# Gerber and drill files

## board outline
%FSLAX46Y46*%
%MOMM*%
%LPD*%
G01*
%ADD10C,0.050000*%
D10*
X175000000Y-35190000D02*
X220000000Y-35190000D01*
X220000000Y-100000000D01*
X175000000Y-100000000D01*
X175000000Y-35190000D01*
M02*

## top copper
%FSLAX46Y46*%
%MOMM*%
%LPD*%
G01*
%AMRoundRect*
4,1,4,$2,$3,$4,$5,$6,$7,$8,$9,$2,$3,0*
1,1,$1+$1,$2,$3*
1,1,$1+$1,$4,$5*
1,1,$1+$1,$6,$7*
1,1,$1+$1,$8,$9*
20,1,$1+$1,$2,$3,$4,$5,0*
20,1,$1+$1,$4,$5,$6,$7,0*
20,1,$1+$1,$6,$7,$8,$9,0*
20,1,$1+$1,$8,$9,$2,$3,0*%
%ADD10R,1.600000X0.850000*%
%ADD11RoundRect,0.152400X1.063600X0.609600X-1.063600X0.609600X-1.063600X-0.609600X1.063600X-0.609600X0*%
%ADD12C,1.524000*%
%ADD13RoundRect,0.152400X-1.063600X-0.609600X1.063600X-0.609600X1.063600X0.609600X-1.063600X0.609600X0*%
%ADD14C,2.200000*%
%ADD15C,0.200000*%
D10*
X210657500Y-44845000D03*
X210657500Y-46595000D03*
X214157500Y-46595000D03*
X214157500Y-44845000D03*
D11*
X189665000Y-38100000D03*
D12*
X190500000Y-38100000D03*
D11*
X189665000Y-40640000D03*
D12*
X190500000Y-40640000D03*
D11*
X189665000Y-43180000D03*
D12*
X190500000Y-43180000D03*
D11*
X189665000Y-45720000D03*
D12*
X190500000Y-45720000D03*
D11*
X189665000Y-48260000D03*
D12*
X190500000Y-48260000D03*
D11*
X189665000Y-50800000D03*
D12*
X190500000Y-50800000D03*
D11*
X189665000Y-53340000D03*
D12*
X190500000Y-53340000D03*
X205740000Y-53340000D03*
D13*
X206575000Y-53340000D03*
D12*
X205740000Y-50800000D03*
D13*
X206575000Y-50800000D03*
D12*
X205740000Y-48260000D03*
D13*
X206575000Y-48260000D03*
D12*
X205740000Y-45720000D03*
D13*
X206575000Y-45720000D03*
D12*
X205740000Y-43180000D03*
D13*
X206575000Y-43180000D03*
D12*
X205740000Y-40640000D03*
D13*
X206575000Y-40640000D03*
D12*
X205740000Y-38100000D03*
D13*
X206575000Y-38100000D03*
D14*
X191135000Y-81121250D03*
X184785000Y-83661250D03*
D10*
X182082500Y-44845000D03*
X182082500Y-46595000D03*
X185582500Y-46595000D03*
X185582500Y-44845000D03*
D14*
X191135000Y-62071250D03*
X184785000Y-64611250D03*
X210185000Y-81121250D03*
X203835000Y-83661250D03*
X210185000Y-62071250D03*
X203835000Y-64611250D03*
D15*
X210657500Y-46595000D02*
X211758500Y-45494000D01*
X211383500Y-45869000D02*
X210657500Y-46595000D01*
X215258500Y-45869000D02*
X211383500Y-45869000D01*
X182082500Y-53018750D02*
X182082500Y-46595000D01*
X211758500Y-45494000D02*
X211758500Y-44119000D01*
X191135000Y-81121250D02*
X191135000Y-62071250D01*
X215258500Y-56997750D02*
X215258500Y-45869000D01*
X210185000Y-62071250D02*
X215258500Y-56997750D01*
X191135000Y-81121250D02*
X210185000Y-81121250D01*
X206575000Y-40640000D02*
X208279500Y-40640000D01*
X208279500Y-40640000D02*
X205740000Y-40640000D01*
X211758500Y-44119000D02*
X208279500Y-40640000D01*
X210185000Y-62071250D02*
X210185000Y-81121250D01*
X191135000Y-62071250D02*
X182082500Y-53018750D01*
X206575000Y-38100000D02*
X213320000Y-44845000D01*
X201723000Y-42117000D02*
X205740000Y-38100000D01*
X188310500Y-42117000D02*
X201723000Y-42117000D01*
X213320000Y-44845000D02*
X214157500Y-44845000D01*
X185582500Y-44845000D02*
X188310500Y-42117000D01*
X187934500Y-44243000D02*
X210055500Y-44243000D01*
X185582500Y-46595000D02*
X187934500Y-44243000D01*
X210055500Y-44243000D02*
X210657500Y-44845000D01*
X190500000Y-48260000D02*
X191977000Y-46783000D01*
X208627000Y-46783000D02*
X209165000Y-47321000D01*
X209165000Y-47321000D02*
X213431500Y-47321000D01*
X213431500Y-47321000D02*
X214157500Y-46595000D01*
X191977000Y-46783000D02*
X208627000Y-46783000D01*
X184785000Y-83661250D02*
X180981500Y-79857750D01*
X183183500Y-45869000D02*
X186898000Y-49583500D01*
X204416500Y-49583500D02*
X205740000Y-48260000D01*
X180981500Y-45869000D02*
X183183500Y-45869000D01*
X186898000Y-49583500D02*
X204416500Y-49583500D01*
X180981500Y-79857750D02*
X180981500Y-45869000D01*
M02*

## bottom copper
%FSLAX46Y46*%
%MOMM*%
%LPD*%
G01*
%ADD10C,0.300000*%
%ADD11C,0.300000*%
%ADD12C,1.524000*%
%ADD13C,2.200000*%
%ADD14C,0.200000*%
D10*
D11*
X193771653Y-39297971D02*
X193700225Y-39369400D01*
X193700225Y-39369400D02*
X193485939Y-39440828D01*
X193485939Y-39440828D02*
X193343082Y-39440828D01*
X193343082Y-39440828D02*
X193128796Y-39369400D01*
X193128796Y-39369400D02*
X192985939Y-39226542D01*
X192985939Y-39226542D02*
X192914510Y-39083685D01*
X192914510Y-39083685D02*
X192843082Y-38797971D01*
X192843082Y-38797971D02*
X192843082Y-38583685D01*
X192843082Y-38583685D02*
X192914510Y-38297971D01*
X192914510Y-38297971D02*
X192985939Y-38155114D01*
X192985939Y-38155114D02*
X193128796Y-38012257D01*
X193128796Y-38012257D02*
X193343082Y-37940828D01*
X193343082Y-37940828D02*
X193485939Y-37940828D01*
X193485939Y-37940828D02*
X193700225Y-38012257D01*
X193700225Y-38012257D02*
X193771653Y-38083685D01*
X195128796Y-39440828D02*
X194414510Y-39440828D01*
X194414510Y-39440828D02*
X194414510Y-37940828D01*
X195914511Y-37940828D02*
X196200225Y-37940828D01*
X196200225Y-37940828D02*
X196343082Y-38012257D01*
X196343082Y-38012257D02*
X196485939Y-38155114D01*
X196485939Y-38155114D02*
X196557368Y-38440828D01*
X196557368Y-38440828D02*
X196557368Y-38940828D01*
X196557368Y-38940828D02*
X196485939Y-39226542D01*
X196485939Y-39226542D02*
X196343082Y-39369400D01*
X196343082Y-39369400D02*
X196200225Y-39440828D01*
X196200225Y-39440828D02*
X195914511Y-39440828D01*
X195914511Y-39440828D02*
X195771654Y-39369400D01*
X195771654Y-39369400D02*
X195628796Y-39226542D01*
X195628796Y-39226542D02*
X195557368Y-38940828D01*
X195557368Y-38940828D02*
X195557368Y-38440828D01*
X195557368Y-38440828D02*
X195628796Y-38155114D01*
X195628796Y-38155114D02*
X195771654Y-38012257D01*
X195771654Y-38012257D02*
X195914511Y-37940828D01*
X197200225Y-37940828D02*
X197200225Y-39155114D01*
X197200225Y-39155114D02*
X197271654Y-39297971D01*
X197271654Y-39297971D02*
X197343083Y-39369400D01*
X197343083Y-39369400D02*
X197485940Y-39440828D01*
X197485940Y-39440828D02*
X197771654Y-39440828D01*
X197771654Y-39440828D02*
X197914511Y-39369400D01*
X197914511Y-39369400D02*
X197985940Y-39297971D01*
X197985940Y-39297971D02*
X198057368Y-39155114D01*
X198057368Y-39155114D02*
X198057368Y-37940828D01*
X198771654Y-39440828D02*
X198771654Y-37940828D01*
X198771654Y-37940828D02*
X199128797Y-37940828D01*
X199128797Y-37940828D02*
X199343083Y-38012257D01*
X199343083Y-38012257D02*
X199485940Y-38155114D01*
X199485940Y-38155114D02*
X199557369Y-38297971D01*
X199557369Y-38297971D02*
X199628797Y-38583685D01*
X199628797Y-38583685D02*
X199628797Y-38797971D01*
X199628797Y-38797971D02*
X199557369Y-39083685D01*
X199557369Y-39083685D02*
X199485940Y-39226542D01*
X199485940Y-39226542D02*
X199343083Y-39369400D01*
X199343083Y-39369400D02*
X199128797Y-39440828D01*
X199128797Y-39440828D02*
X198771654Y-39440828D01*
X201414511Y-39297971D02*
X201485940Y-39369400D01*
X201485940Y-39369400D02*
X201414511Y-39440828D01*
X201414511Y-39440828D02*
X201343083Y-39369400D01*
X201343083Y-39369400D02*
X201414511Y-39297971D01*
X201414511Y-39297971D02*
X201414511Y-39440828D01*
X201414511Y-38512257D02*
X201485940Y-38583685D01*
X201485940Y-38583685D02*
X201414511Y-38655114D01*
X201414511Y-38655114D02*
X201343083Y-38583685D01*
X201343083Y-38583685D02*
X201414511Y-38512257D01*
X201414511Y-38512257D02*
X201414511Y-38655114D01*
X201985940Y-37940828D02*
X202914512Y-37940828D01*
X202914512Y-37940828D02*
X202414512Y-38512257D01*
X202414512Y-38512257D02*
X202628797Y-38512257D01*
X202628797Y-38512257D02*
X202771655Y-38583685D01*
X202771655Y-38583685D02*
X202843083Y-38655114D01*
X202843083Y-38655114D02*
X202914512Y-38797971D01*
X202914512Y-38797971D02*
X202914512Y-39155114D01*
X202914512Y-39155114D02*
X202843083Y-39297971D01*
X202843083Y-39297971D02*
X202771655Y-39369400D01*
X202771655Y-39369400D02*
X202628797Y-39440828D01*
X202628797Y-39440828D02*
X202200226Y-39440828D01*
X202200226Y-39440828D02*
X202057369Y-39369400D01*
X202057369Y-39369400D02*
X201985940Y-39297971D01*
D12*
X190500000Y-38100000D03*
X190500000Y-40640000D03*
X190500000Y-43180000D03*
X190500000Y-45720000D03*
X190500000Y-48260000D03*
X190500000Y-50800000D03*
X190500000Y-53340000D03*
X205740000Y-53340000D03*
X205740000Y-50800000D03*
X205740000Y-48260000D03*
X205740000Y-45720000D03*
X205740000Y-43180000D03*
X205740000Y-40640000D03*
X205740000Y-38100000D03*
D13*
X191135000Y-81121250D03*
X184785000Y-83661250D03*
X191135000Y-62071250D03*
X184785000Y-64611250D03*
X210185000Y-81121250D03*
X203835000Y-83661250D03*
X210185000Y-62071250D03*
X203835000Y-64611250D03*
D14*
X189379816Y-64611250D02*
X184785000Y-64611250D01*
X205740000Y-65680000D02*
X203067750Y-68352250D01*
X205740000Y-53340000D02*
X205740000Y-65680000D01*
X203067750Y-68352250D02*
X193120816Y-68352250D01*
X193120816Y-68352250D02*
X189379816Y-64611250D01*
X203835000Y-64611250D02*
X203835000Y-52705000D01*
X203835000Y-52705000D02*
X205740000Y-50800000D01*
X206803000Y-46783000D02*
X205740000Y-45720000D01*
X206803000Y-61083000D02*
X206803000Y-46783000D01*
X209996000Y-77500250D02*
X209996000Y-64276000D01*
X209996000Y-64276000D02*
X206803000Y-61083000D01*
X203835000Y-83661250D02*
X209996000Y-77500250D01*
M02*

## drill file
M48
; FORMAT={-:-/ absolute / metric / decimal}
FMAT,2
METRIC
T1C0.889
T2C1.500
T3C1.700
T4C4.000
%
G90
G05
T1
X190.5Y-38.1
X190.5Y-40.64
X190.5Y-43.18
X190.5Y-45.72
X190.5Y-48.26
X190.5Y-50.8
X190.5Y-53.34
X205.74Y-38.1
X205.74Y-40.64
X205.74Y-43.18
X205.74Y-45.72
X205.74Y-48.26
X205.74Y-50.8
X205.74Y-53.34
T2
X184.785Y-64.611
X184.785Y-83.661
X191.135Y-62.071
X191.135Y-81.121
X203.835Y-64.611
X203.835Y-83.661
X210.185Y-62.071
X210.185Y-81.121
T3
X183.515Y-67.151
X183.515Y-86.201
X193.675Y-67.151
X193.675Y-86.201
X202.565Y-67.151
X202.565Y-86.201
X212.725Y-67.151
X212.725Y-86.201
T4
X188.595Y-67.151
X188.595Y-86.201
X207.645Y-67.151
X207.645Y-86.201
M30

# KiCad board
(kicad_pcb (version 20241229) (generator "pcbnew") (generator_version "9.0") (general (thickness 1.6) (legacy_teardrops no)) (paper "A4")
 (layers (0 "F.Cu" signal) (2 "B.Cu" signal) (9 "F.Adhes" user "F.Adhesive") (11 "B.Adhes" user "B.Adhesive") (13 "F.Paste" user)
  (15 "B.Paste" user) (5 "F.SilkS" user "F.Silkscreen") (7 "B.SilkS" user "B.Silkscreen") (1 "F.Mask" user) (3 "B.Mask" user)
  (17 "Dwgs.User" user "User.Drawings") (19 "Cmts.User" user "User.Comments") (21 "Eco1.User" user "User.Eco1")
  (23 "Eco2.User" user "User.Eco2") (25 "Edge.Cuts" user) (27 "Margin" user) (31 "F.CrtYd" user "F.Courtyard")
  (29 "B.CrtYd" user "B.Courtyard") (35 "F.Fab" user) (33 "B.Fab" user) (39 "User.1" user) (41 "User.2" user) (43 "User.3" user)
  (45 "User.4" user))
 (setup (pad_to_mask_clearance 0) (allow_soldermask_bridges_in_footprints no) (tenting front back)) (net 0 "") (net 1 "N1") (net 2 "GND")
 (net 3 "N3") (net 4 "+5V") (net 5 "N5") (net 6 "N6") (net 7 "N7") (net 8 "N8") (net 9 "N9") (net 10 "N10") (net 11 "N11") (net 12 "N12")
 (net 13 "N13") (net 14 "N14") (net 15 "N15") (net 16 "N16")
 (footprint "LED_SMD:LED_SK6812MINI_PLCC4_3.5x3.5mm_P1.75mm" (layer "F.Cu") (at 212.4075 45.72)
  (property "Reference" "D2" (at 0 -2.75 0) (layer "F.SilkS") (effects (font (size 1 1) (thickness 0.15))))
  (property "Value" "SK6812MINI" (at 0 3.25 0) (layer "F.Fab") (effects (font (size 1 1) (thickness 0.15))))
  (pad "1" smd rect (at -1.75 -0.875) (size 1.6 0.85) (layers "F.Cu" "F.Mask" "F.Paste") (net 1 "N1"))
  (pad "2" smd rect (at -1.75 0.875) (size 1.6 0.85) (layers "F.Cu" "F.Mask" "F.Paste") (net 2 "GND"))
  (pad "3" smd rect (at 1.75 0.875) (size 1.6 0.85) (layers "F.Cu" "F.Mask" "F.Paste") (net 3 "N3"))
  (pad "4" smd rect (at 1.75 -0.875) (size 1.6 0.85) (layers "F.Cu" "F.Mask" "F.Paste") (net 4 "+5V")))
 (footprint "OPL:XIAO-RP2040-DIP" (layer "F.Cu") (at 198.12 45.72)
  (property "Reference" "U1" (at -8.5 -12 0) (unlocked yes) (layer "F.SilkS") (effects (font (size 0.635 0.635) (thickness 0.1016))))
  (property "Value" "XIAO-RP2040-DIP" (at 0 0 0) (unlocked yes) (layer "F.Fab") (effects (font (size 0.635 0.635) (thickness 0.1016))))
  (pad "1" smd roundrect (at -8.455 -7.62 180) (size 2.432 1.524) (layers "F.Cu" "F.Mask") (roundrect_rratio 0.1) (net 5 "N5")
   (thermal_bridge_angle 45))
  (pad "1" thru_hole circle (at -7.62 -7.62 180) (size 1.524 1.524) (drill 0.889) (layers "*.Cu" "*.Mask") (remove_unused_layers no)
   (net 5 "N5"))
  (pad "2" smd roundrect (at -8.455 -5.08 180) (size 2.432 1.524) (layers "F.Cu" "F.Mask") (roundrect_rratio 0.1) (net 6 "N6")
   (thermal_bridge_angle 45))
  (pad "2" thru_hole circle (at -7.62 -5.08 180) (size 1.524 1.524) (drill 0.889) (layers "*.Cu" "*.Mask") (remove_unused_layers no)
   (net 6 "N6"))
  (pad "3" smd roundrect (at -8.455 -2.54 180) (size 2.432 1.524) (layers "F.Cu" "F.Mask") (roundrect_rratio 0.1) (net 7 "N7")
   (thermal_bridge_angle 45))
  (pad "3" thru_hole circle (at -7.62 -2.54 180) (size 1.524 1.524) (drill 0.889) (layers "*.Cu" "*.Mask") (remove_unused_layers no)
   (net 7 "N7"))
  (pad "4" smd roundrect (at -8.455 0 180) (size 2.432 1.524) (layers "F.Cu" "F.Mask") (roundrect_rratio 0.1) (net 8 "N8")
   (thermal_bridge_angle 45))
  (pad "4" thru_hole circle (at -7.62 0 180) (size 1.524 1.524) (drill 0.889) (layers "*.Cu" "*.Mask") (remove_unused_layers no)
   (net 8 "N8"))
  (pad "5" smd roundrect (at -8.455 2.54 180) (size 2.432 1.524) (layers "F.Cu" "F.Mask") (roundrect_rratio 0.1) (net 3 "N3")
   (thermal_bridge_angle 45))
  (pad "5" thru_hole circle (at -7.62 2.54 180) (size 1.524 1.524) (drill 0.889) (layers "*.Cu" "*.Mask") (remove_unused_layers no)
   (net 3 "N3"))
  (pad "6" smd roundrect (at -8.455 5.08 180) (size 2.432 1.524) (layers "F.Cu" "F.Mask") (roundrect_rratio 0.1) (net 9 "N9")
   (thermal_bridge_angle 45))
  (pad "6" thru_hole circle (at -7.62 5.08 180) (size 1.524 1.524) (drill 0.889) (layers "*.Cu" "*.Mask") (remove_unused_layers no)
   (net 9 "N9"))
  (pad "7" smd roundrect (at -8.455 7.62 180) (size 2.432 1.524) (layers "F.Cu" "F.Mask") (roundrect_rratio 0.1) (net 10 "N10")
   (thermal_bridge_angle 45))
  (pad "7" thru_hole circle (at -7.62 7.62 180) (size 1.524 1.524) (drill 0.889) (layers "*.Cu" "*.Mask") (remove_unused_layers no)
   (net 10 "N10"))
  (pad "8" thru_hole circle (at 7.62 7.62) (size 1.524 1.524) (drill 0.889) (layers "*.Cu" "*.Mask") (remove_unused_layers no)
   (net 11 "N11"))
  (pad "8" smd roundrect (at 8.455 7.62) (size 2.432 1.524) (layers "F.Cu" "F.Mask") (roundrect_rratio 0.1) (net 11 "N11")
   (thermal_bridge_angle 45))
  (pad "9" thru_hole circle (at 7.62 5.08) (size 1.524 1.524) (drill 0.889) (layers "*.Cu" "*.Mask") (remove_unused_layers no)
   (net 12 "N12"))
  (pad "9" smd roundrect (at 8.455 5.08) (size 2.432 1.524) (layers "F.Cu" "F.Mask") (roundrect_rratio 0.1) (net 12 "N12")
   (thermal_bridge_angle 45))
  (pad "10" thru_hole circle (at 7.62 2.54) (size 1.524 1.524) (drill 0.889) (layers "*.Cu" "*.Mask") (remove_unused_layers no)
   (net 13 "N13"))
  (pad "10" smd roundrect (at 8.455 2.54) (size 2.432 1.524) (layers "F.Cu" "F.Mask") (roundrect_rratio 0.1) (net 13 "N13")
   (thermal_bridge_angle 45))
  (pad "11" thru_hole circle (at 7.62 0) (size 1.524 1.524) (drill 0.889) (layers "*.Cu" "*.Mask") (remove_unused_layers no) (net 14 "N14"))
  (pad "11" smd roundrect (at 8.455 0) (size 2.432 1.524) (layers "F.Cu" "F.Mask") (roundrect_rratio 0.1) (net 14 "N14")
   (thermal_bridge_angle 45))
  (pad "12" thru_hole circle (at 7.62 -2.54) (size 1.524 1.524) (drill 0.889) (layers "*.Cu" "*.Mask") (remove_unused_layers no)
   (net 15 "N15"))
  (pad "12" smd roundrect (at 8.455 -2.54) (size 2.432 1.524) (layers "F.Cu" "F.Mask") (roundrect_rratio 0.1) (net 15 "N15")
   (thermal_bridge_angle 45))
  (pad "13" thru_hole circle (at 7.62 -5.08) (size 1.524 1.524) (drill 0.889) (layers "*.Cu" "*.Mask") (remove_unused_layers no)
   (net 2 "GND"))
  (pad "13" smd roundrect (at 8.455 -5.08) (size 2.432 1.524) (layers "F.Cu" "F.Mask") (roundrect_rratio 0.1) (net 2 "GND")
   (thermal_bridge_angle 45))
  (pad "14" thru_hole circle (at 7.62 -7.62) (size 1.524 1.524) (drill 0.889) (layers "*.Cu" "*.Mask") (remove_unused_layers no)
   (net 4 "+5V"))
  (pad "14" smd roundrect (at 8.455 -7.62) (size 2.432 1.524) (layers "F.Cu" "F.Mask") (roundrect_rratio 0.1) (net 4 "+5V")
   (thermal_bridge_angle 45)))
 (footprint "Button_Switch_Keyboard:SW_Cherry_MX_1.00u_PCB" (layer "F.Cu") (at 191.135 81.12125)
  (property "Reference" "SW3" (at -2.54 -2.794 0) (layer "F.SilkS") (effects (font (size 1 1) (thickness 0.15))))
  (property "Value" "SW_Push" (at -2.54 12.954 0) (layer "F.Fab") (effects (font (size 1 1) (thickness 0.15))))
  (pad "" np_thru_hole circle (at -7.62 5.08) (size 1.7 1.7) (drill 1.7) (layers "*.Cu" "*.Mask"))
  (pad "" np_thru_hole circle (at -2.54 5.08) (size 4 4) (drill 4) (layers "*.Cu" "*.Mask"))
  (pad "" np_thru_hole circle (at 2.54 5.08) (size 1.7 1.7) (drill 1.7) (layers "*.Cu" "*.Mask"))
  (pad "1" thru_hole circle (at 0 0) (size 2.2 2.2) (drill 1.5) (layers "*.Cu" "*.Mask") (remove_unused_layers no) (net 2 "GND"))
  (pad "2" thru_hole circle (at -6.35 2.54) (size 2.2 2.2) (drill 1.5) (layers "*.Cu" "*.Mask") (remove_unused_layers no) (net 13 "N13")))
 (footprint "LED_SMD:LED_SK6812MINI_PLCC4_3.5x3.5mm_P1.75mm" (layer "F.Cu") (at 183.8325 45.72)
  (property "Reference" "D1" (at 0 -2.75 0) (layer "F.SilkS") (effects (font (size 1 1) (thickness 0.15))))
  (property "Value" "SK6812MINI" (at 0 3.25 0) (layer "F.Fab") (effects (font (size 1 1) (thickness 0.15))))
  (pad "1" smd rect (at -1.75 -0.875) (size 1.6 0.85) (layers "F.Cu" "F.Mask" "F.Paste") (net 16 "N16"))
  (pad "2" smd rect (at -1.75 0.875) (size 1.6 0.85) (layers "F.Cu" "F.Mask" "F.Paste") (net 2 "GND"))
  (pad "3" smd rect (at 1.75 0.875) (size 1.6 0.85) (layers "F.Cu" "F.Mask" "F.Paste") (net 1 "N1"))
  (pad "4" smd rect (at 1.75 -0.875) (size 1.6 0.85) (layers "F.Cu" "F.Mask" "F.Paste") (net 4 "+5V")))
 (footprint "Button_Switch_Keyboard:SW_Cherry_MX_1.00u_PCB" (layer "F.Cu") (at 191.135 62.07125)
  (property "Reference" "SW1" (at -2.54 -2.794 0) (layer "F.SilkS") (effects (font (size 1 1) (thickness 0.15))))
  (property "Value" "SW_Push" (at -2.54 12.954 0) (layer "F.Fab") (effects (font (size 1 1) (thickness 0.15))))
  (pad "" np_thru_hole circle (at -7.62 5.08) (size 1.7 1.7) (drill 1.7) (layers "*.Cu" "*.Mask"))
  (pad "" np_thru_hole circle (at -2.54 5.08) (size 4 4) (drill 4) (layers "*.Cu" "*.Mask"))
  (pad "" np_thru_hole circle (at 2.54 5.08) (size 1.7 1.7) (drill 1.7) (layers "*.Cu" "*.Mask"))
  (pad "1" thru_hole circle (at 0 0) (size 2.2 2.2) (drill 1.5) (layers "*.Cu" "*.Mask") (remove_unused_layers no) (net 2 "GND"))
  (pad "2" thru_hole circle (at -6.35 2.54) (size 2.2 2.2) (drill 1.5) (layers "*.Cu" "*.Mask") (remove_unused_layers no) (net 11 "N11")))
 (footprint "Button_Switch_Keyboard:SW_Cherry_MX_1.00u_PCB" (layer "F.Cu") (at 210.185 81.12125)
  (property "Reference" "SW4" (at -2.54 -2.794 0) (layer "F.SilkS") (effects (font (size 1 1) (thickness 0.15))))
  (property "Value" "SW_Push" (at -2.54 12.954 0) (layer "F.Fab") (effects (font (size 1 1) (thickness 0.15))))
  (pad "" np_thru_hole circle (at -7.62 5.08) (size 1.7 1.7) (drill 1.7) (layers "*.Cu" "*.Mask"))
  (pad "" np_thru_hole circle (at -2.54 5.08) (size 4 4) (drill 4) (layers "*.Cu" "*.Mask"))
  (pad "" np_thru_hole circle (at 2.54 5.08) (size 1.7 1.7) (drill 1.7) (layers "*.Cu" "*.Mask"))
  (pad "1" thru_hole circle (at 0 0) (size 2.2 2.2) (drill 1.5) (layers "*.Cu" "*.Mask") (remove_unused_layers no) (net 2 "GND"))
  (pad "2" thru_hole circle (at -6.35 2.54) (size 2.2 2.2) (drill 1.5) (layers "*.Cu" "*.Mask") (remove_unused_layers no) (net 14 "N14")))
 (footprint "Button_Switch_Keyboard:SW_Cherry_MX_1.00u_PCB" (layer "F.Cu") (at 210.185 62.07125)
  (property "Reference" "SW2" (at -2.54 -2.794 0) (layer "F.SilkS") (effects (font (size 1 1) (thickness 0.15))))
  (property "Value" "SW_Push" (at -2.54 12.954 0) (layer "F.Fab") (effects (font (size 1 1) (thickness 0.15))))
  (pad "" np_thru_hole circle (at -7.62 5.08) (size 1.7 1.7) (drill 1.7) (layers "*.Cu" "*.Mask"))
  (pad "" np_thru_hole circle (at -2.54 5.08) (size 4 4) (drill 4) (layers "*.Cu" "*.Mask"))
  (pad "" np_thru_hole circle (at 2.54 5.08) (size 1.7 1.7) (drill 1.7) (layers "*.Cu" "*.Mask"))
  (pad "1" thru_hole circle (at 0 0) (size 2.2 2.2) (drill 1.5) (layers "*.Cu" "*.Mask") (remove_unused_layers no) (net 2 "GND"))
  (pad "2" thru_hole circle (at -6.35 2.54) (size 2.2 2.2) (drill 1.5) (layers "*.Cu" "*.Mask") (remove_unused_layers no) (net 12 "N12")))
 (gr_rect (start 175 35.19) (end 220 100) (stroke (width 0.05) (type default)) (fill no) (layer "Edge.Cuts"))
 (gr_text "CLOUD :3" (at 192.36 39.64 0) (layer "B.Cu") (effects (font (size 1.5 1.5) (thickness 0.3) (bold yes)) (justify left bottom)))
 (segment (start 210.6575 46.595) (end 211.7585 45.494) (width 0.2) (layer "F.Cu") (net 2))
 (segment (start 211.3835 45.869) (end 210.6575 46.595) (width 0.2) (layer "F.Cu") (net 2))
 (segment (start 215.2585 45.869) (end 211.3835 45.869) (width 0.2) (layer "F.Cu") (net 2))
 (segment (start 182.0825 53.01875) (end 182.0825 46.595) (width 0.2) (layer "F.Cu") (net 2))
 (segment (start 211.7585 45.494) (end 211.7585 44.119) (width 0.2) (layer "F.Cu") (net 2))
 (segment (start 191.135 81.12125) (end 191.135 62.07125) (width 0.2) (layer "F.Cu") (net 2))
 (segment (start 215.2585 56.99775) (end 215.2585 45.869) (width 0.2) (layer "F.Cu") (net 2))
 (segment (start 210.185 62.07125) (end 215.2585 56.99775) (width 0.2) (layer "F.Cu") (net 2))
 (segment (start 191.135 81.12125) (end 210.185 81.12125) (width 0.2) (layer "F.Cu") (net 2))
 (segment (start 206.575 40.64) (end 208.2795 40.64) (width 0.2) (layer "F.Cu") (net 2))
 (segment (start 208.2795 40.64) (end 205.74 40.64) (width 0.2) (layer "F.Cu") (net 2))
 (segment (start 211.7585 44.119) (end 208.2795 40.64) (width 0.2) (layer "F.Cu") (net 2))
 (segment (start 210.185 62.07125) (end 210.185 81.12125) (width 0.2) (layer "F.Cu") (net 2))
 (segment (start 191.135 62.07125) (end 182.0825 53.01875) (width 0.2) (layer "F.Cu") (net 2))
 (segment (start 206.575 38.1) (end 213.32 44.845) (width 0.2) (layer "F.Cu") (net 4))
 (segment (start 201.723 42.117) (end 205.74 38.1) (width 0.2) (layer "F.Cu") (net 4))
 (segment (start 188.3105 42.117) (end 201.723 42.117) (width 0.2) (layer "F.Cu") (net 4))
 (segment (start 213.32 44.845) (end 214.1575 44.845) (width 0.2) (layer "F.Cu") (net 4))
 (segment (start 185.5825 44.845) (end 188.3105 42.117) (width 0.2) (layer "F.Cu") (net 4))
 (segment (start 187.9345 44.243) (end 210.0555 44.243) (width 0.2) (layer "F.Cu") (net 1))
 (segment (start 185.5825 46.595) (end 187.9345 44.243) (width 0.2) (layer "F.Cu") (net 1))
 (segment (start 210.0555 44.243) (end 210.6575 44.845) (width 0.2) (layer "F.Cu") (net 1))
 (segment (start 190.5 48.26) (end 191.977 46.783) (width 0.2) (layer "F.Cu") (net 3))
 (segment (start 208.627 46.783) (end 209.165 47.321) (width 0.2) (layer "F.Cu") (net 3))
 (segment (start 209.165 47.321) (end 213.4315 47.321) (width 0.2) (layer "F.Cu") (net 3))
 (segment (start 213.4315 47.321) (end 214.1575 46.595) (width 0.2) (layer "F.Cu") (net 3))
 (segment (start 191.977 46.783) (end 208.627 46.783) (width 0.2) (layer "F.Cu") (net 3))
 (segment (start 189.379816 64.61125) (end 184.785 64.61125) (width 0.2) (layer "B.Cu") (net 11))
 (segment (start 205.74 65.68) (end 203.06775 68.35225) (width 0.2) (layer "B.Cu") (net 11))
 (segment (start 205.74 53.34) (end 205.74 65.68) (width 0.2) (layer "B.Cu") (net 11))
 (segment (start 203.06775 68.35225) (end 193.120816 68.35225) (width 0.2) (layer "B.Cu") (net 11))
 (segment (start 193.120816 68.35225) (end 189.379816 64.61125) (width 0.2) (layer "B.Cu") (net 11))
 (segment (start 203.835 64.61125) (end 203.835 52.705) (width 0.2) (layer "B.Cu") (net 12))
 (segment (start 203.835 52.705) (end 205.74 50.8) (width 0.2) (layer "B.Cu") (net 12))
 (segment (start 184.785 83.66125) (end 180.9815 79.85775) (width 0.2) (layer "F.Cu") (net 13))
 (segment (start 183.1835 45.869) (end 186.898 49.5835) (width 0.2) (layer "F.Cu") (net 13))
 (segment (start 204.4165 49.5835) (end 205.74 48.26) (width 0.2) (layer "F.Cu") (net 13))
 (segment (start 180.9815 45.869) (end 183.1835 45.869) (width 0.2) (layer "F.Cu") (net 13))
 (segment (start 186.898 49.5835) (end 204.4165 49.5835) (width 0.2) (layer "F.Cu") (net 13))
 (segment (start 180.9815 79.85775) (end 180.9815 45.869) (width 0.2) (layer "F.Cu") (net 13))
 (segment (start 206.803 46.783) (end 205.74 45.72) (width 0.2) (layer "B.Cu") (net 14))
 (segment (start 206.803 61.083) (end 206.803 46.783) (width 0.2) (layer "B.Cu") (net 14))
 (segment (start 209.996 77.50025) (end 209.996 64.276) (width 0.2) (layer "B.Cu") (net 14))
 (segment (start 209.996 64.276) (end 206.803 61.083) (width 0.2) (layer "B.Cu") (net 14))
 (segment (start 203.835 83.66125) (end 209.996 77.50025) (width 0.2) (layer "B.Cu") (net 14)))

